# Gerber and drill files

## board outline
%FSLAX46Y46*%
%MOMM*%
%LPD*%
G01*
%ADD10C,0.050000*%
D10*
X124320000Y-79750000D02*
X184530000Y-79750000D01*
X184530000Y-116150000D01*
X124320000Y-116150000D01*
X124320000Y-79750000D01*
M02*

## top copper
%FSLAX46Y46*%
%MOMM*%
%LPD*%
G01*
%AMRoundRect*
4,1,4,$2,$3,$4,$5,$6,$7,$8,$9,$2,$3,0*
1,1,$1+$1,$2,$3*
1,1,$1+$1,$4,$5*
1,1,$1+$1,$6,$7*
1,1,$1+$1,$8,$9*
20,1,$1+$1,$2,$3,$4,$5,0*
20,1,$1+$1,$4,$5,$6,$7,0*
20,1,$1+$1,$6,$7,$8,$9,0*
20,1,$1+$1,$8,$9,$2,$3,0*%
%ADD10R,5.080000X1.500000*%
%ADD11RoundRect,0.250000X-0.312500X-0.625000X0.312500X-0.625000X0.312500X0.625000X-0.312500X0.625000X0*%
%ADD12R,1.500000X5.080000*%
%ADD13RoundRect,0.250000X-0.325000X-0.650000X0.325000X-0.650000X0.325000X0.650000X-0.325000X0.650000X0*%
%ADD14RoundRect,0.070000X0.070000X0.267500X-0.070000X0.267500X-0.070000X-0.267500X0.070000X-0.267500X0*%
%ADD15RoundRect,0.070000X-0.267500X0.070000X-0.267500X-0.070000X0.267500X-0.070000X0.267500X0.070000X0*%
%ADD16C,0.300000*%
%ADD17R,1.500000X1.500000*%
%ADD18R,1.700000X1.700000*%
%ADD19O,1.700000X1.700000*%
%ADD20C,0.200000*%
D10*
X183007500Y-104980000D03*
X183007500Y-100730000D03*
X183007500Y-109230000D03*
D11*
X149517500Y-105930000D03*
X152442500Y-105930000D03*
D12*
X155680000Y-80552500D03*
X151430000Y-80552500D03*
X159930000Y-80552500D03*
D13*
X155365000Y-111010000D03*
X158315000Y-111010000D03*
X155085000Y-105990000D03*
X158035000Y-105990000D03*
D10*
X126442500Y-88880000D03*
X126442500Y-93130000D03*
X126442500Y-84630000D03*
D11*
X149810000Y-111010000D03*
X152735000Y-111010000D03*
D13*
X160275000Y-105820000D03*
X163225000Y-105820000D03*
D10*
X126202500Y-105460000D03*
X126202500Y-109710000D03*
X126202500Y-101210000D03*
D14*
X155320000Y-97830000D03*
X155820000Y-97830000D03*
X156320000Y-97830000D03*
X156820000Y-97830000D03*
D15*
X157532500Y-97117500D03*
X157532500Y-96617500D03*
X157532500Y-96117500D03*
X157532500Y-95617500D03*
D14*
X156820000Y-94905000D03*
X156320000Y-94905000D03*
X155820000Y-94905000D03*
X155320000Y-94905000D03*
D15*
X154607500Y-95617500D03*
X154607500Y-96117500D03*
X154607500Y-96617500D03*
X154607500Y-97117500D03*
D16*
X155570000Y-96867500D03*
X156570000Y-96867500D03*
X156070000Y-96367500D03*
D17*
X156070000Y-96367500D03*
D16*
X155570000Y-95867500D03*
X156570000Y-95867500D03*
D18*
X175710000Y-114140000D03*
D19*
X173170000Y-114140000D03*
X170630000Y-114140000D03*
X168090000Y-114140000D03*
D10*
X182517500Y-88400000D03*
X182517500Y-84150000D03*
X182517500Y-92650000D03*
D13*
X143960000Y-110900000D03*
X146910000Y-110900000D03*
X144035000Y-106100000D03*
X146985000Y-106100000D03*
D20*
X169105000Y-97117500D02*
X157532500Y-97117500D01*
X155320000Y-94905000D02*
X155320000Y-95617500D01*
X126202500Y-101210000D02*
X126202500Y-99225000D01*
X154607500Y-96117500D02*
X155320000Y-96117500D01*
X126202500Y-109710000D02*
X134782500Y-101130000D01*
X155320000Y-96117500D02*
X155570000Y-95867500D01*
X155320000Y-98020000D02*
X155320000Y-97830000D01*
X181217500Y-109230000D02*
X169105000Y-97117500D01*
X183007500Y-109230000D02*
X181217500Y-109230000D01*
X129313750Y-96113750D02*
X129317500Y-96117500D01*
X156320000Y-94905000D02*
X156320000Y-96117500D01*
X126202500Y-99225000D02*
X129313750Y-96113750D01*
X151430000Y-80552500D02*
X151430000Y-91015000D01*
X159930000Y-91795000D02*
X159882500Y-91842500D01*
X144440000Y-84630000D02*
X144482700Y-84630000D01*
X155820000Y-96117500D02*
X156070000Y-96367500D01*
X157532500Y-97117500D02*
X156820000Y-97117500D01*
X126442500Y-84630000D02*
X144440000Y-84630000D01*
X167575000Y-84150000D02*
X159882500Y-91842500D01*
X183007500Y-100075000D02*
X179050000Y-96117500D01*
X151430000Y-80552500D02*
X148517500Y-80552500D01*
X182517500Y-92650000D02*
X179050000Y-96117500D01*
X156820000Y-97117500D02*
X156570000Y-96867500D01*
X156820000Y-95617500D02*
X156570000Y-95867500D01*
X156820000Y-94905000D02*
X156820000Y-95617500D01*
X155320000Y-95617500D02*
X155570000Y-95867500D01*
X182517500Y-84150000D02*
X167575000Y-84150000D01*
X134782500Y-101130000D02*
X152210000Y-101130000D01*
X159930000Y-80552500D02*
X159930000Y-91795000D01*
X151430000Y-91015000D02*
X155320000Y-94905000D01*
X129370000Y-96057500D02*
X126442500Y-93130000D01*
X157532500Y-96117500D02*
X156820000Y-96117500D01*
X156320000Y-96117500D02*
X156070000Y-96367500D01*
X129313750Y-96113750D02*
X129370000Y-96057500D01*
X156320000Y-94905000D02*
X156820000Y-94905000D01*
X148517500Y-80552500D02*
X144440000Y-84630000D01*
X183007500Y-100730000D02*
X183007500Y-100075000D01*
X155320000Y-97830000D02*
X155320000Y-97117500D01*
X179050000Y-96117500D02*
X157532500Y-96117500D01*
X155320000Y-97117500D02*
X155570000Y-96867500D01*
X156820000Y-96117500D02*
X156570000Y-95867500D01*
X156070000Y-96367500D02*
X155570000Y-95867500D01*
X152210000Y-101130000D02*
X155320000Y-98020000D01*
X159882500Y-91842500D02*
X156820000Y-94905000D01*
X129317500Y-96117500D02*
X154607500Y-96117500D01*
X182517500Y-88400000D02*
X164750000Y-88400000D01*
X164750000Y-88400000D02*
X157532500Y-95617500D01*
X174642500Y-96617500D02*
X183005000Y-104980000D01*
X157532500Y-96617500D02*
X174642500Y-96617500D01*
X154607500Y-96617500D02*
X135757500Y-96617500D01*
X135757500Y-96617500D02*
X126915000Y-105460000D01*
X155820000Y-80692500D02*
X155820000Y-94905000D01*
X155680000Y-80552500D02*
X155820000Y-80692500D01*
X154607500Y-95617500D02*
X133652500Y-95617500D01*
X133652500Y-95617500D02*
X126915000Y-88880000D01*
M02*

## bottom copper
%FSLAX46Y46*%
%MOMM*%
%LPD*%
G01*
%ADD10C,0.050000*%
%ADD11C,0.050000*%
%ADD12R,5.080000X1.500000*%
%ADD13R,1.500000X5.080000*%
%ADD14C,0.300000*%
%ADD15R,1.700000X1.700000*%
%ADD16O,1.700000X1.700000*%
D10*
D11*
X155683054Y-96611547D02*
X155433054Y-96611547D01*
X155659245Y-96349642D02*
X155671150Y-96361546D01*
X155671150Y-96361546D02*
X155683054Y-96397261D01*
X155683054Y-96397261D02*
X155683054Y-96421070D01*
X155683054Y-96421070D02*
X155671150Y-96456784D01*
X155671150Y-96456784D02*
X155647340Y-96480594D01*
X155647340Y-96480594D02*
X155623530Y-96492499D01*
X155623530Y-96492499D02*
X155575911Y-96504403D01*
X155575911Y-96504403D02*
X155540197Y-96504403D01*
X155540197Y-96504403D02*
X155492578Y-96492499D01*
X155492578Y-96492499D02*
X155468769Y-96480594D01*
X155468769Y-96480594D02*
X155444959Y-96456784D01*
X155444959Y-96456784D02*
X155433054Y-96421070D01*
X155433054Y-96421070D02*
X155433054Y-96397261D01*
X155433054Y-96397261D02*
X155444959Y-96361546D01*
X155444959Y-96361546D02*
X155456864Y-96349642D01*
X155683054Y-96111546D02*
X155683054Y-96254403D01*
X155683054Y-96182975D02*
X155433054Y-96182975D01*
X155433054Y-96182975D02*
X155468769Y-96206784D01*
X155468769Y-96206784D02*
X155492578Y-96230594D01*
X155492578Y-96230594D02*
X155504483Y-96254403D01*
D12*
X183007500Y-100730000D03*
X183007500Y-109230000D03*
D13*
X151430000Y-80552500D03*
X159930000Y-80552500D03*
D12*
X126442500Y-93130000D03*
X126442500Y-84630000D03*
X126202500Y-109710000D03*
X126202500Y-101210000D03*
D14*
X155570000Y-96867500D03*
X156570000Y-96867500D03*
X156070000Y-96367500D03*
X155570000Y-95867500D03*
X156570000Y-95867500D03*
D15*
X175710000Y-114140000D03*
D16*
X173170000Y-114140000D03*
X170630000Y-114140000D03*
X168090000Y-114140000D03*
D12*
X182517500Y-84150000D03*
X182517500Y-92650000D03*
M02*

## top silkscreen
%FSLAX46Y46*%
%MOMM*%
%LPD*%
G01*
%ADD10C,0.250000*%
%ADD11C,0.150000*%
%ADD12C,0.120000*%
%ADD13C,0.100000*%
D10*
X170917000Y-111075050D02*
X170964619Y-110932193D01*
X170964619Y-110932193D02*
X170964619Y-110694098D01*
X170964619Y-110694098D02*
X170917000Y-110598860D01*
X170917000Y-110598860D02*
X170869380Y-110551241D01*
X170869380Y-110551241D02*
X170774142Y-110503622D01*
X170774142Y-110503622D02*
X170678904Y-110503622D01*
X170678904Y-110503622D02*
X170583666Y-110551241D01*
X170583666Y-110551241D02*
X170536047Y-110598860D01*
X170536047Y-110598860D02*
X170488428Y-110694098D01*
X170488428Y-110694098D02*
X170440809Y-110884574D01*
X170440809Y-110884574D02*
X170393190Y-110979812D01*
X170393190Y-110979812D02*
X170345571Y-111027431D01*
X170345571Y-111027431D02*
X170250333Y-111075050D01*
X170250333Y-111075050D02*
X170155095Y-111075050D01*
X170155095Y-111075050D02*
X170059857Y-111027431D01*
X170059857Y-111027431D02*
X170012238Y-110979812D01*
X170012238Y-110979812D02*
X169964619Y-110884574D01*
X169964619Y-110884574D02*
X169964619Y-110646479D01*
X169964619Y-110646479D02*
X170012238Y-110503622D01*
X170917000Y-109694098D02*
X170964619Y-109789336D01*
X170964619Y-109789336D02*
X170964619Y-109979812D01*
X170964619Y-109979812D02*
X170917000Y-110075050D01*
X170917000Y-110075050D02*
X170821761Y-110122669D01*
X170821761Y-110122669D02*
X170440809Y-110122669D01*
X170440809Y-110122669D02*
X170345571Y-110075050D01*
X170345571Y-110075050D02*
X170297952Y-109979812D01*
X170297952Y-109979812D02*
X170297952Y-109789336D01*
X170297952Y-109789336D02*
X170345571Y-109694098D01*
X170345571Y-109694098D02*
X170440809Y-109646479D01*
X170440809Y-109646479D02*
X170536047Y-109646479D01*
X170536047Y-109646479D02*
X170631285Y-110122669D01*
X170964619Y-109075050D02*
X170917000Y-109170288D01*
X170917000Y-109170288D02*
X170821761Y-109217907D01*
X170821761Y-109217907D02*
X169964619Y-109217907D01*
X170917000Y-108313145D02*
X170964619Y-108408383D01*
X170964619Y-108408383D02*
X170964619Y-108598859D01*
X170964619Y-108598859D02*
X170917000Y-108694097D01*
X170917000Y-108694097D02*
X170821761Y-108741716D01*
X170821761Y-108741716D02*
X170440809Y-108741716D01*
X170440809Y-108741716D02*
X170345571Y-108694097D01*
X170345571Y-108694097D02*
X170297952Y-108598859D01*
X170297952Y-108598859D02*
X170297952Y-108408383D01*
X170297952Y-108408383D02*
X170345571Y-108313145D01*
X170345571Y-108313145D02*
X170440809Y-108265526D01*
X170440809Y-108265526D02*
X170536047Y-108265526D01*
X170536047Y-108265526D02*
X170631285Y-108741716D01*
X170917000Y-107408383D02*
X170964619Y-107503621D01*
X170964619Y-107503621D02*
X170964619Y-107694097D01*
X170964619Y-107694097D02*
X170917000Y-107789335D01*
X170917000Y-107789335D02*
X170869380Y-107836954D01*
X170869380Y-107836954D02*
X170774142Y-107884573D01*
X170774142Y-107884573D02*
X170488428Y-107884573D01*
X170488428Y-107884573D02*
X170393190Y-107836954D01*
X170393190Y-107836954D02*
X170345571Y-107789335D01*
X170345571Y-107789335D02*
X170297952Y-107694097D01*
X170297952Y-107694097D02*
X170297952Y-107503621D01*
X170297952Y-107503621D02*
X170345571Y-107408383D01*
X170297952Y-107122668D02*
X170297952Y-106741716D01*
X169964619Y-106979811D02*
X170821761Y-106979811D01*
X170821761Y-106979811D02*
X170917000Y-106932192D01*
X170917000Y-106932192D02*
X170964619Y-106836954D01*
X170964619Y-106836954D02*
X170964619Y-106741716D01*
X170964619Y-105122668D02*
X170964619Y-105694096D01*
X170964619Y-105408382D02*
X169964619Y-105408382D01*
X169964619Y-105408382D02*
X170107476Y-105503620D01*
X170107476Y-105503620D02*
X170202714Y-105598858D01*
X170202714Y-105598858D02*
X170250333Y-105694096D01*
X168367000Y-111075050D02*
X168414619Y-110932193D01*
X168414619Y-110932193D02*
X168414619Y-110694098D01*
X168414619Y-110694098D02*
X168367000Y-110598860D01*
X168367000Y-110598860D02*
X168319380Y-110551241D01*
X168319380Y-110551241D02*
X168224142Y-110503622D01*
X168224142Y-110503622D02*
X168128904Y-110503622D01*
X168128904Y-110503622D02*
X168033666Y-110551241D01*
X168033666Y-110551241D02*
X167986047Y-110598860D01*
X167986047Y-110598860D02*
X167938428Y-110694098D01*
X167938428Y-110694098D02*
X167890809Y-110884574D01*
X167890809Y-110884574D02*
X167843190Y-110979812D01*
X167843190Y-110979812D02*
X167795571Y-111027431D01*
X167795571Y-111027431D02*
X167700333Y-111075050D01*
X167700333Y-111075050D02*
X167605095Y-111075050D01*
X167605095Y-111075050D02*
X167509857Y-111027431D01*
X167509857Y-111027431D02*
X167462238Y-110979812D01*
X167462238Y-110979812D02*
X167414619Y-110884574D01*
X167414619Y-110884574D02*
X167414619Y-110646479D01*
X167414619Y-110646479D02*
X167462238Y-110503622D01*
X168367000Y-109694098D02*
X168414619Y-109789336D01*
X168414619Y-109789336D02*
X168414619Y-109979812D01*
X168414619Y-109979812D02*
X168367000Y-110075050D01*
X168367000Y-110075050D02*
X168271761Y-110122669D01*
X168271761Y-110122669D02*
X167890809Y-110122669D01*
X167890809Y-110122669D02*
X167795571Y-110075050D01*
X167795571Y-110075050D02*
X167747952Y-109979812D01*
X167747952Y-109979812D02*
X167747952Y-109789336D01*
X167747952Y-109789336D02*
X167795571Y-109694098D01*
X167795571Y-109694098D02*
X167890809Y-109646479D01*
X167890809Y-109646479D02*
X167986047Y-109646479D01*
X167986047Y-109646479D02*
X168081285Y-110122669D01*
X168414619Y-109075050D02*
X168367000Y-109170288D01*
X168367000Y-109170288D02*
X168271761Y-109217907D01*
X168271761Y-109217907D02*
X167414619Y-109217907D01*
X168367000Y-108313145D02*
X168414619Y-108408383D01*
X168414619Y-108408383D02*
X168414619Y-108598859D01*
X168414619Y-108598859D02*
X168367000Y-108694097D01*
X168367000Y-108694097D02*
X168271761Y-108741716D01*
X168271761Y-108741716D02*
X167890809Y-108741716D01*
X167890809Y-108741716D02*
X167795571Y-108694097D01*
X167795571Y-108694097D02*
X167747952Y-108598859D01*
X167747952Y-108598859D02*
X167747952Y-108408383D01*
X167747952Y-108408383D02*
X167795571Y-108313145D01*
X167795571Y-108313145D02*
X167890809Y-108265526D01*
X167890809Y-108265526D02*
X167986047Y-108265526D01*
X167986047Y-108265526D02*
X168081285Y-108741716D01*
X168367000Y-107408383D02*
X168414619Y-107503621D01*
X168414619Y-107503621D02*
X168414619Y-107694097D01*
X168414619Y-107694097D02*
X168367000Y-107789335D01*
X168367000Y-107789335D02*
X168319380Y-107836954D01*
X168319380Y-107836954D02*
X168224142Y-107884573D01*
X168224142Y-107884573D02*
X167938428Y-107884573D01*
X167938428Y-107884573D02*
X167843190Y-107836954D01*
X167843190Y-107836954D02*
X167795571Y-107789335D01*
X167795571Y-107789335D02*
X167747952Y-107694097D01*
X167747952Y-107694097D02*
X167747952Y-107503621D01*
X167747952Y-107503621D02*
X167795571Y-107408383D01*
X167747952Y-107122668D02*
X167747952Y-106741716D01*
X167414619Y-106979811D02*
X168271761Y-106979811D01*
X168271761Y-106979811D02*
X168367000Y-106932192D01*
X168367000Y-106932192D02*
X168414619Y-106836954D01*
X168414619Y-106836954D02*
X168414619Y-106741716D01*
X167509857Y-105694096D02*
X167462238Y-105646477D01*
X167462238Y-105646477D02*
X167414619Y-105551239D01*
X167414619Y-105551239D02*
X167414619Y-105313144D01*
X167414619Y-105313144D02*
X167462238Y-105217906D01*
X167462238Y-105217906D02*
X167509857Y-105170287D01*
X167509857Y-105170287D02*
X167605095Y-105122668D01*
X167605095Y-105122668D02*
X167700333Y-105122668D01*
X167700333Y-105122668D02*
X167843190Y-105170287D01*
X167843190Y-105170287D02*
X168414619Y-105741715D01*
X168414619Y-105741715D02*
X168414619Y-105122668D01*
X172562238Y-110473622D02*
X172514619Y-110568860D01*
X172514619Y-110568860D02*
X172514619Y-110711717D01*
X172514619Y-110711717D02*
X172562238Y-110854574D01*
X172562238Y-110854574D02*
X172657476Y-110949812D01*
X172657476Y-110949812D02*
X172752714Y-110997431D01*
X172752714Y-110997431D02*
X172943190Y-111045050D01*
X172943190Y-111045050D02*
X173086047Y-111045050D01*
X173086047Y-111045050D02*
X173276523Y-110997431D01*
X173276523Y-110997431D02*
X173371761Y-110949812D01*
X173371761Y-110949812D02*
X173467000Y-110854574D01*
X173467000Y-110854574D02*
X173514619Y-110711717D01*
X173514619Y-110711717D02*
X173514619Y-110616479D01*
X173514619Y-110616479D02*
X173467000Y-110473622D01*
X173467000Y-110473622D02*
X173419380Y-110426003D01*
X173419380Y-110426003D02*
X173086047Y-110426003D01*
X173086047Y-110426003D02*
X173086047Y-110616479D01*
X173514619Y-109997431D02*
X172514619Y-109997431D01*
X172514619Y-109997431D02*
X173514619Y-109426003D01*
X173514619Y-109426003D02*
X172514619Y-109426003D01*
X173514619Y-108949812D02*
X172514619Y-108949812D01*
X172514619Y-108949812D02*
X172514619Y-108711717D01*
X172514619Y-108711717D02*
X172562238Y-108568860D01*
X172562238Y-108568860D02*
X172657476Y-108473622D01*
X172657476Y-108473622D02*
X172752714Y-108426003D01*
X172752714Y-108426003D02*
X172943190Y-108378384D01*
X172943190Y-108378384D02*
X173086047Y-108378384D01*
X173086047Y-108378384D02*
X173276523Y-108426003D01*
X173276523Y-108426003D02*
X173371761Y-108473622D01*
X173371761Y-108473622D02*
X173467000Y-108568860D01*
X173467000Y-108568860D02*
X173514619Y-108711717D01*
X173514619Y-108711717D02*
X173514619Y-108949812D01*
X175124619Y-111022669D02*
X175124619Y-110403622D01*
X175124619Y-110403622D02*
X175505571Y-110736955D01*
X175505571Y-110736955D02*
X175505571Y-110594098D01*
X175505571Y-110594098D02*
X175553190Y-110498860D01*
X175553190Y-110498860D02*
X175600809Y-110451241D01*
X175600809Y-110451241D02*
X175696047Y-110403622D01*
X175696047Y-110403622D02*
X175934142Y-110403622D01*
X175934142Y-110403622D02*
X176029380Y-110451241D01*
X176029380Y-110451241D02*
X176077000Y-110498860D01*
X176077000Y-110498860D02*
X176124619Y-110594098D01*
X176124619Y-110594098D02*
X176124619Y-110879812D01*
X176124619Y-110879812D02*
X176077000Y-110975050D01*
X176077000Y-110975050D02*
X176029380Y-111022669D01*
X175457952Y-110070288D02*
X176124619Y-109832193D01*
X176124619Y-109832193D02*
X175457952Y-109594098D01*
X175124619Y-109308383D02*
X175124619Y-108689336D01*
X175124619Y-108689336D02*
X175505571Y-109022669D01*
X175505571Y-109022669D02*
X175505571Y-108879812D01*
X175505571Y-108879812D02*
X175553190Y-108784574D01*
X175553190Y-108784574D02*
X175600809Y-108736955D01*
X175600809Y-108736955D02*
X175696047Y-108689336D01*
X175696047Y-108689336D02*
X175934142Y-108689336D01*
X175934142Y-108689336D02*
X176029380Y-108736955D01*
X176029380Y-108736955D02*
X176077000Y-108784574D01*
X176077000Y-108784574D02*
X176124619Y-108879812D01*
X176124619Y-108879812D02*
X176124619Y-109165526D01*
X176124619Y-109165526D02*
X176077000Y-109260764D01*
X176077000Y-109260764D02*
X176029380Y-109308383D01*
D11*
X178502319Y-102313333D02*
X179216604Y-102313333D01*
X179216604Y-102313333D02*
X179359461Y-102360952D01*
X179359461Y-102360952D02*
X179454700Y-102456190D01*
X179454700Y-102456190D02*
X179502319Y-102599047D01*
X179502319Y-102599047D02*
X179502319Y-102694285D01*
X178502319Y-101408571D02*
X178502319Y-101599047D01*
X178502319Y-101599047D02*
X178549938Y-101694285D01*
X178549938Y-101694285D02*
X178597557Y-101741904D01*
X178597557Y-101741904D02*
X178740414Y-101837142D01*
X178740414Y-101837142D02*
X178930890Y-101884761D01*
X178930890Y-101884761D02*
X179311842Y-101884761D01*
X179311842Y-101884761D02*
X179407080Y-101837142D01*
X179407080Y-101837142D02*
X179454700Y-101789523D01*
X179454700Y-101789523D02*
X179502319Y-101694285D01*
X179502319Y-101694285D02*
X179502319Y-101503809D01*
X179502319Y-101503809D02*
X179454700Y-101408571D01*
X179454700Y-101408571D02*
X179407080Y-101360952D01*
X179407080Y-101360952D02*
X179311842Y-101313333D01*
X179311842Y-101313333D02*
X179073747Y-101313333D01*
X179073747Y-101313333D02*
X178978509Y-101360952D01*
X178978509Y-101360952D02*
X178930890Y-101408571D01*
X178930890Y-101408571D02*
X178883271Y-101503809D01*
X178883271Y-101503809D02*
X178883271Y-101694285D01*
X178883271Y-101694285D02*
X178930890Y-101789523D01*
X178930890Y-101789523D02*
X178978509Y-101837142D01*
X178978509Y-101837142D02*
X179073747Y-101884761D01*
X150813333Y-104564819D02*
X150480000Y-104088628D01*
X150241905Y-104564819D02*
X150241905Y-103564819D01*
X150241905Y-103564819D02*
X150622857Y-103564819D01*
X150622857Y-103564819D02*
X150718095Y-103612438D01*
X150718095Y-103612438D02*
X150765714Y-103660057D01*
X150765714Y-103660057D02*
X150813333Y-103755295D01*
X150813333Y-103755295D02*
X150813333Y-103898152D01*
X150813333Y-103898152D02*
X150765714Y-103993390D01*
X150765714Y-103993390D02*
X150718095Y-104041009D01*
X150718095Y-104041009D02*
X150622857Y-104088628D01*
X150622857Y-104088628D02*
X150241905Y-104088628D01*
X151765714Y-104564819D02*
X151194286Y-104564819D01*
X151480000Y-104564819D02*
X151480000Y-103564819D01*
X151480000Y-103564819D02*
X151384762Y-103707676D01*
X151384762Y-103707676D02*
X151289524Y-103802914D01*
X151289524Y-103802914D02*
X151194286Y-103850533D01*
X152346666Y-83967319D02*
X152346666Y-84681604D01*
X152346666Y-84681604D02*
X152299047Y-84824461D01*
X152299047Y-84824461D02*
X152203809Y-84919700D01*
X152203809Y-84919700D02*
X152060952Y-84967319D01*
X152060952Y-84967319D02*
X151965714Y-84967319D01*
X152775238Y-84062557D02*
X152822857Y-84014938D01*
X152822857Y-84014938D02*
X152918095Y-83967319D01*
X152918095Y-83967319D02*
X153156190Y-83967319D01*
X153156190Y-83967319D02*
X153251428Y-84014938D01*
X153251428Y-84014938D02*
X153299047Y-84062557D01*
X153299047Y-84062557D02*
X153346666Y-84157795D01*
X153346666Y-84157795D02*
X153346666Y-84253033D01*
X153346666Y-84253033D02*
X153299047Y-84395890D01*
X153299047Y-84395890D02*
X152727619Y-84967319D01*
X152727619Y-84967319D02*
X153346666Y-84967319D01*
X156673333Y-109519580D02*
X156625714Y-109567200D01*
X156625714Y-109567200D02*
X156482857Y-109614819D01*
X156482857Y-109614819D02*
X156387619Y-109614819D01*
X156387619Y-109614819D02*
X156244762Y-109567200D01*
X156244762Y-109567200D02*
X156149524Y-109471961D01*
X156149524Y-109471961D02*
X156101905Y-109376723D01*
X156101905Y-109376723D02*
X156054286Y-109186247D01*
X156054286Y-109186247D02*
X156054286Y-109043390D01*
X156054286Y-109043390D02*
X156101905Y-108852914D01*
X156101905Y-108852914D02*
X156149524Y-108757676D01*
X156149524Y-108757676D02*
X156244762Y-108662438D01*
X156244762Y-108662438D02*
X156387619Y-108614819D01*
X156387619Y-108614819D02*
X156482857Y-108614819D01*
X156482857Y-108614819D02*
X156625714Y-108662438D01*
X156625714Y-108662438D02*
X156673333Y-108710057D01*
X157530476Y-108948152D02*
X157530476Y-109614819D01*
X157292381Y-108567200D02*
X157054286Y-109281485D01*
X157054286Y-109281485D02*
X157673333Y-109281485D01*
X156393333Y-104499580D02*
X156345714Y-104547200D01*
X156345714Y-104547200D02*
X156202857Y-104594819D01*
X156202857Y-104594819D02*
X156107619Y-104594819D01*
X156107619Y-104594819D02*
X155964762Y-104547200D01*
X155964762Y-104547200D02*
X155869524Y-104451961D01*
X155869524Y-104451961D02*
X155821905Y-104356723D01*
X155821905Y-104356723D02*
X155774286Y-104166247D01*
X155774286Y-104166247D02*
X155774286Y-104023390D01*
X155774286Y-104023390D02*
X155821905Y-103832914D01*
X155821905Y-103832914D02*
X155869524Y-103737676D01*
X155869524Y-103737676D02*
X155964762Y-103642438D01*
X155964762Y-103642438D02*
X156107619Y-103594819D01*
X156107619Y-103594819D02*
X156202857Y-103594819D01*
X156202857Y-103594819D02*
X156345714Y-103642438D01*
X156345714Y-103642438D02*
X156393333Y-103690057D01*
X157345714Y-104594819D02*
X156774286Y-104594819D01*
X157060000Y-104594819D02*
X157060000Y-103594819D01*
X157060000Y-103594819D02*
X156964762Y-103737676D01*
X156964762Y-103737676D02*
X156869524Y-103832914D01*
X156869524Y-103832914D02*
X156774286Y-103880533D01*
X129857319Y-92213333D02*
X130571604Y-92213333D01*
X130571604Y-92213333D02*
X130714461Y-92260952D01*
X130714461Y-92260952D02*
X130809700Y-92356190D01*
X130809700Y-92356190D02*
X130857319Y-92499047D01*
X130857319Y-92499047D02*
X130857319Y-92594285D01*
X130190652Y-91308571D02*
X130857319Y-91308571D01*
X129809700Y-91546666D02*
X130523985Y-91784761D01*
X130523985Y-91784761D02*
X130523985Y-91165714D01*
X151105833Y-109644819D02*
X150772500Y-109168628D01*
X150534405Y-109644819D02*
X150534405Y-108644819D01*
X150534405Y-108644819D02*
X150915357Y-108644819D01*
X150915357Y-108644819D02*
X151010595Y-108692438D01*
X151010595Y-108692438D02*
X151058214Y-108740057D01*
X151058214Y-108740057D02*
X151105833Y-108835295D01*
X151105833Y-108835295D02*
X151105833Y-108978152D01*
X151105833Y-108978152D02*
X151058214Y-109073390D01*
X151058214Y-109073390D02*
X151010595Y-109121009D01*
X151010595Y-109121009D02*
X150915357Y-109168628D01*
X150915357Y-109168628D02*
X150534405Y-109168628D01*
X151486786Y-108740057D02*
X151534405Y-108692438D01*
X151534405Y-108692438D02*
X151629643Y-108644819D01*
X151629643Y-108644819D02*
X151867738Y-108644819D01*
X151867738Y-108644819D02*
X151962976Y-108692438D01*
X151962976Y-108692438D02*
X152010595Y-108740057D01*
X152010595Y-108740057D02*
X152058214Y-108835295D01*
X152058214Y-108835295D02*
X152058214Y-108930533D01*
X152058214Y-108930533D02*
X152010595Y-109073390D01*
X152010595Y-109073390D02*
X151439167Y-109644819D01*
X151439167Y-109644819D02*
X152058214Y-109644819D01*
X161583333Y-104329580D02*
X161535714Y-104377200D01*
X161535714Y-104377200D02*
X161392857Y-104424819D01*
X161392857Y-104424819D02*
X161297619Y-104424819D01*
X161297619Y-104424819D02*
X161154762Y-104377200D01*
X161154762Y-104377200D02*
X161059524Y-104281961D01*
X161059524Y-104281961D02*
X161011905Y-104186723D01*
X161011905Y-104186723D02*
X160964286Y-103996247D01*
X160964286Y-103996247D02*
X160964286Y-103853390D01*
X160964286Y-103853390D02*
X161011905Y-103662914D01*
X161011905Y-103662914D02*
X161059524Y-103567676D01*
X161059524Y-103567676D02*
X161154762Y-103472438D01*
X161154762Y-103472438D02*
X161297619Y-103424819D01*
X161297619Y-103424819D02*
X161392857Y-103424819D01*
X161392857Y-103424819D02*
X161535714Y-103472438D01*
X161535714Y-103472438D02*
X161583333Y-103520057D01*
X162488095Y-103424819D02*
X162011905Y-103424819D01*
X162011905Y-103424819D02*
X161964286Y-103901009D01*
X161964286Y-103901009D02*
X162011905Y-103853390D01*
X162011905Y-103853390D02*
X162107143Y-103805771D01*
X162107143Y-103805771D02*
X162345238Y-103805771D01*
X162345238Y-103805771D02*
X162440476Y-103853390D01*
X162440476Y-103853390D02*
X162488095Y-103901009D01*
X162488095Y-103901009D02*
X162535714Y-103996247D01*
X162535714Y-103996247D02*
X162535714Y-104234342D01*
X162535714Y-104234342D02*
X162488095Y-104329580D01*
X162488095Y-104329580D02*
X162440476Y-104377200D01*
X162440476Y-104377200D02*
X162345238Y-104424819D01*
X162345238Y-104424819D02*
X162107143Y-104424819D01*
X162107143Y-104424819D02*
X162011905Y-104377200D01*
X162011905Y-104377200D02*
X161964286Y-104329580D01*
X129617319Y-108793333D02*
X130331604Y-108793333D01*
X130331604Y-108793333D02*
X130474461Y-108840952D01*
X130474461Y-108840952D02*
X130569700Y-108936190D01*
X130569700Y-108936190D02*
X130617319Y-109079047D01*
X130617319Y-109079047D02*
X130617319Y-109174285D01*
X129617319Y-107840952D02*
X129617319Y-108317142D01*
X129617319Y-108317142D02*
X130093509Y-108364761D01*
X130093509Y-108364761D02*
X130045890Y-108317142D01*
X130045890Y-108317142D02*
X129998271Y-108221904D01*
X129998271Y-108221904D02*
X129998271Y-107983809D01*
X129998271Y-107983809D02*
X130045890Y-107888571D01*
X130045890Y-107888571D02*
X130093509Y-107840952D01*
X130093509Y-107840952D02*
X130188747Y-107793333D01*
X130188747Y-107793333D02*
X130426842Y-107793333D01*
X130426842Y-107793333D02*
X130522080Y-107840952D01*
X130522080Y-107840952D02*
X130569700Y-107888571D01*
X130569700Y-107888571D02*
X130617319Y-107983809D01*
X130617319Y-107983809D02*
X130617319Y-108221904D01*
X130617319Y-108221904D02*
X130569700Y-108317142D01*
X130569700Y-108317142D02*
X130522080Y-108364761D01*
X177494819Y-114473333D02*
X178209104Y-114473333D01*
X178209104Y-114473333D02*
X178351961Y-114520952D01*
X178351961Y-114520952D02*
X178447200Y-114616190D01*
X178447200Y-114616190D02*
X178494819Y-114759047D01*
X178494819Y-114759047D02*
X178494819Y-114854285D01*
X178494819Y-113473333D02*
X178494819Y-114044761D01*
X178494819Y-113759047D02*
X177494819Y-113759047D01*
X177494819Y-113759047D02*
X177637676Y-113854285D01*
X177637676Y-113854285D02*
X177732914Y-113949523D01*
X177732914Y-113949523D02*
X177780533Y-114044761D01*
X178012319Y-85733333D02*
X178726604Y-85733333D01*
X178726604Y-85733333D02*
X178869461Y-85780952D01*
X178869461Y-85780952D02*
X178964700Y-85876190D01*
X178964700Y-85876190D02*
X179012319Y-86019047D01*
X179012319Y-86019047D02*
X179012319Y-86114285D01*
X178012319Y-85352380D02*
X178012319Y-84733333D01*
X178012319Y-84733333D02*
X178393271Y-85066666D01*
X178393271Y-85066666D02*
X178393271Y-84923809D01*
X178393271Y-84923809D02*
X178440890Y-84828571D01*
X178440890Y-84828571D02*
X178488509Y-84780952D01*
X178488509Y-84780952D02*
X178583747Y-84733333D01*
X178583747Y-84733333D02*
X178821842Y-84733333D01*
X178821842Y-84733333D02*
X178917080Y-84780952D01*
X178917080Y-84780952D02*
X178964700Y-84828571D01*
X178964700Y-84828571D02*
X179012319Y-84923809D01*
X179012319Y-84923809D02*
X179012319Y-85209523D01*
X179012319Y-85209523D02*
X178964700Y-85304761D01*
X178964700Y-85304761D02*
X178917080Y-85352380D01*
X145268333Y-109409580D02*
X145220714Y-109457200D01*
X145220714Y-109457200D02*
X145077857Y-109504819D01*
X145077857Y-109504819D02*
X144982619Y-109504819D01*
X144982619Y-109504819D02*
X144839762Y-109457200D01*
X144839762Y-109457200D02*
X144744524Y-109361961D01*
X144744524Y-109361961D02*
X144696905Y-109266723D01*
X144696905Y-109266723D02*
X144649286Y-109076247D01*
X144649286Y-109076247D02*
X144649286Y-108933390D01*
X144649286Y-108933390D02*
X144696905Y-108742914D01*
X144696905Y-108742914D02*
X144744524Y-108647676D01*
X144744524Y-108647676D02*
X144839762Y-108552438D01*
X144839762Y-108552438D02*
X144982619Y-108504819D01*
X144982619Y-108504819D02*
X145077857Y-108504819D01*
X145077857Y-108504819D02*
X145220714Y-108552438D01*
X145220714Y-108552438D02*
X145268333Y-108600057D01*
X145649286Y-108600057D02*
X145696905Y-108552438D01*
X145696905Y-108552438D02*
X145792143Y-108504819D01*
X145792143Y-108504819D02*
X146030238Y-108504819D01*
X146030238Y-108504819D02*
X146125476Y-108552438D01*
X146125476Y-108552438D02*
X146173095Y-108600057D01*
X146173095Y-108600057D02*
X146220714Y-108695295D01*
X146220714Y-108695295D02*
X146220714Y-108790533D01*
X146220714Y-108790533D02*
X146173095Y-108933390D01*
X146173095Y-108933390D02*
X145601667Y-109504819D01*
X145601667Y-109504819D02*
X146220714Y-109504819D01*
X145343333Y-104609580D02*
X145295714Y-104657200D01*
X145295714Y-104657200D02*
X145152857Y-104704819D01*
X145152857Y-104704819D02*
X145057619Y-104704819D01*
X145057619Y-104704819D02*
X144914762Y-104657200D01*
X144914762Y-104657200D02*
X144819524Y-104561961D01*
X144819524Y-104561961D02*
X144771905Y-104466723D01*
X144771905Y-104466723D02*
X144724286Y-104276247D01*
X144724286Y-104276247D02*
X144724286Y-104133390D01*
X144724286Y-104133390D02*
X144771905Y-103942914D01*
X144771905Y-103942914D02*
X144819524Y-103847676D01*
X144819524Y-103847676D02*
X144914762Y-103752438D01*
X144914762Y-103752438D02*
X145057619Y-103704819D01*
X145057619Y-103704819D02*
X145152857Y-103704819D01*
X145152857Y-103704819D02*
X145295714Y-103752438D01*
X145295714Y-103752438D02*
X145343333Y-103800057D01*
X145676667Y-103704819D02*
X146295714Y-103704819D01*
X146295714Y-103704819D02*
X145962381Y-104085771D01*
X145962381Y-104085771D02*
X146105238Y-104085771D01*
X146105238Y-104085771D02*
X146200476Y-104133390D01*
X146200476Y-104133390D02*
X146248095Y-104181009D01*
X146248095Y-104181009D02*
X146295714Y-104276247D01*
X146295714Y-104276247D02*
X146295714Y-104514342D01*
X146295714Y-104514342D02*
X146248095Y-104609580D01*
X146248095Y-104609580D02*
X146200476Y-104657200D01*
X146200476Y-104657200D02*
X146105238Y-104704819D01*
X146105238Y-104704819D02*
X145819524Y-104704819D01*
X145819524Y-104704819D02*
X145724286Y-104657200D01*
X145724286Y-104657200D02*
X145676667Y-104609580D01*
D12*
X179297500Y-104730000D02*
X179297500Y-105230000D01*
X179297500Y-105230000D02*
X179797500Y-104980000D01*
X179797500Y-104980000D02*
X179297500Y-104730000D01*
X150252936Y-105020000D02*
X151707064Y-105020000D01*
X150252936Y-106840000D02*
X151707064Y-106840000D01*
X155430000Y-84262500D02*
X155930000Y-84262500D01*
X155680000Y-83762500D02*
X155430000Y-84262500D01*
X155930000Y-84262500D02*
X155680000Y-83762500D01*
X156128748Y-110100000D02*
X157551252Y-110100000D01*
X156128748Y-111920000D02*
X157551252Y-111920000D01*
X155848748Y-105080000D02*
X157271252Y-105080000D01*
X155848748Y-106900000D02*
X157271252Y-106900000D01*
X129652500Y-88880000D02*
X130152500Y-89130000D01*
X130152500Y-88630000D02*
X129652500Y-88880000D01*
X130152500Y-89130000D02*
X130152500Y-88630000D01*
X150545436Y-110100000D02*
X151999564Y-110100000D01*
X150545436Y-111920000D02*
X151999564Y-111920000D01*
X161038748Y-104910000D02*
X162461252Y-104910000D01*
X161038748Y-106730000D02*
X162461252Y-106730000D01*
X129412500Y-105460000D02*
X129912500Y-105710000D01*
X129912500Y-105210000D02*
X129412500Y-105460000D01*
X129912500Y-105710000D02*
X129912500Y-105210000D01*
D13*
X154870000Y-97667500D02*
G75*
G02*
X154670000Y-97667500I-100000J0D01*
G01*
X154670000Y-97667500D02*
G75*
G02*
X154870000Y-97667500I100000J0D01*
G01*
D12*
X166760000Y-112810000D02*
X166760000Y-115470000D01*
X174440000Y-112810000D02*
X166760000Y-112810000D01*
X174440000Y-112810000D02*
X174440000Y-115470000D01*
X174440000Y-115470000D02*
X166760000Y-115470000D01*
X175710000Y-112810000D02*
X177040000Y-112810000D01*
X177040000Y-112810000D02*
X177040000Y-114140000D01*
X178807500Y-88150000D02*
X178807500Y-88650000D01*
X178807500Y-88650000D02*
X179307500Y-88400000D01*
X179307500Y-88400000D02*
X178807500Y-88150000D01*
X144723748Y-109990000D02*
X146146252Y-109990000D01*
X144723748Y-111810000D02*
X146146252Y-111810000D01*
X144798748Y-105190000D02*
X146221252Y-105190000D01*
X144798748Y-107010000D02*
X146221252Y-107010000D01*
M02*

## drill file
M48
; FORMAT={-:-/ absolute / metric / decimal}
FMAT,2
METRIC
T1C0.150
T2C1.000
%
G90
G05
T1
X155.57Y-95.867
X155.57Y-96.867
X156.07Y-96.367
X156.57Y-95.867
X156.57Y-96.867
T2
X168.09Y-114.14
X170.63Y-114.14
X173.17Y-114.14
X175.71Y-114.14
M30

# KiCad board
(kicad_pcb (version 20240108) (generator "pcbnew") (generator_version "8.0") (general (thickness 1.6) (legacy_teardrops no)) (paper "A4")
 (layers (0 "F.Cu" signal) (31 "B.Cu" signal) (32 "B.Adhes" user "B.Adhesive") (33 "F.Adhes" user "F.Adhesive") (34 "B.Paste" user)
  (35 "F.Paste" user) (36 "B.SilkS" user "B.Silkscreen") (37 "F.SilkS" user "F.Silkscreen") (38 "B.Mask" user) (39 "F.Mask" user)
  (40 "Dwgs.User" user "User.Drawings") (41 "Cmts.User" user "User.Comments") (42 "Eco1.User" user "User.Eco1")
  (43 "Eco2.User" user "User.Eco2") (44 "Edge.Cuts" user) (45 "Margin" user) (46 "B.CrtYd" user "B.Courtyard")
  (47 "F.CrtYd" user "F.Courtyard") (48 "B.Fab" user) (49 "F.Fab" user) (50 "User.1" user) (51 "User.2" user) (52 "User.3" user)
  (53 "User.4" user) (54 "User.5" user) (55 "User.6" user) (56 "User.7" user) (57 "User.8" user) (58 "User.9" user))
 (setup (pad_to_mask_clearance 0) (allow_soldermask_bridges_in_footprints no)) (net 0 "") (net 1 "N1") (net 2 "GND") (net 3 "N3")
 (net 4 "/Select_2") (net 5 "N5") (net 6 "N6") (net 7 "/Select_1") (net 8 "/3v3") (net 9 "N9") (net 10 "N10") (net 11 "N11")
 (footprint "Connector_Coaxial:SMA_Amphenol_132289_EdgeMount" (layer "F.Cu") (at 183.0075 104.98)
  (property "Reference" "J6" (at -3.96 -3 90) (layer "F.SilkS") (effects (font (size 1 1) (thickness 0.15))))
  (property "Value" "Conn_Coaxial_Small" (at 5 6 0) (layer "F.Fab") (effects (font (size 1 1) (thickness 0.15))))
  (fp_line (start -3.71 -0.25) (end -3.71 0.25) (stroke (width 0.12) (type solid)) (layer "F.SilkS"))
  (fp_line (start -3.71 0.25) (end -3.21 0) (stroke (width 0.12) (type solid)) (layer "F.SilkS"))
  (fp_line (start -3.21 0) (end -3.71 -0.25) (stroke (width 0.12) (type solid)) (layer "F.SilkS"))
  (pad "1" smd rect (at 0 0 90) (size 1.5 5.08) (layers "F.Cu" "F.Paste" "F.Mask") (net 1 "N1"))
  (pad "2" smd rect (at 0 -4.25 90) (size 1.5 5.08) (layers "F.Cu" "F.Paste" "F.Mask") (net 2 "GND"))
  (pad "2" smd rect (at 0 -4.25 90) (size 1.5 5.08) (layers "B.Cu" "B.Paste" "B.Mask") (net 2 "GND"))
  (pad "2" smd rect (at 0 4.25 90) (size 1.5 5.08) (layers "F.Cu" "F.Paste" "F.Mask") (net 2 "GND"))
  (pad "2" smd rect (at 0 4.25 90) (size 1.5 5.08) (layers "B.Cu" "B.Paste" "B.Mask") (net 2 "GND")))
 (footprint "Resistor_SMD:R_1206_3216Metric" (layer "F.Cu") (at 150.98 105.93)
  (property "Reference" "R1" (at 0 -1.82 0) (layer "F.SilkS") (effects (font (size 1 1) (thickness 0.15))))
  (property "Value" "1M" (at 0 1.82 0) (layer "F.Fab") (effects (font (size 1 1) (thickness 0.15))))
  (fp_line (start -0.727064 -0.91) (end 0.727064 -0.91) (stroke (width 0.12) (type solid)) (layer "F.SilkS"))
  (fp_line (start -0.727064 0.91) (end 0.727064 0.91) (stroke (width 0.12) (type solid)) (layer "F.SilkS"))
  (pad "1" smd roundrect (at -1.4625 0) (size 1.125 1.75) (layers "F.Cu" "F.Paste" "F.Mask") (roundrect_rratio 0.222222) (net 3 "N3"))
  (pad "2" smd roundrect (at 1.4625 0) (size 1.125 1.75) (layers "F.Cu" "F.Paste" "F.Mask") (roundrect_rratio 0.222222) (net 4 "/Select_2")))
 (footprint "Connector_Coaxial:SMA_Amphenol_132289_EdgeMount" (layer "F.Cu") (at 155.68 80.5525 90)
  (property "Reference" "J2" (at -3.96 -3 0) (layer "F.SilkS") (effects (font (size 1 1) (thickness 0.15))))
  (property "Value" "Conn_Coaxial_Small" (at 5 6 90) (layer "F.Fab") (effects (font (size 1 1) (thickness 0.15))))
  (fp_line (start -3.71 -0.25) (end -3.71 0.25) (stroke (width 0.12) (type solid)) (layer "F.SilkS"))
  (fp_line (start -3.21 0) (end -3.71 -0.25) (stroke (width 0.12) (type solid)) (layer "F.SilkS"))
  (fp_line (start -3.71 0.25) (end -3.21 0) (stroke (width 0.12) (type solid)) (layer "F.SilkS"))
  (pad "1" smd rect (at 0 0 180) (size 1.5 5.08) (layers "F.Cu" "F.Paste" "F.Mask") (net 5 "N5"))
  (pad "2" smd rect (at 0 -4.25 180) (size 1.5 5.08) (layers "F.Cu" "F.Paste" "F.Mask") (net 2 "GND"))
  (pad "2" smd rect (at 0 -4.25 180) (size 1.5 5.08) (layers "B.Cu" "B.Paste" "B.Mask") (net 2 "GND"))
  (pad "2" smd rect (at 0 4.25 180) (size 1.5 5.08) (layers "F.Cu" "F.Paste" "F.Mask") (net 2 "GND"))
  (pad "2" smd rect (at 0 4.25 180) (size 1.5 5.08) (layers "B.Cu" "B.Paste" "B.Mask") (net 2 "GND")))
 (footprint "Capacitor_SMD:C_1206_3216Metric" (layer "F.Cu") (at 156.84 111.01)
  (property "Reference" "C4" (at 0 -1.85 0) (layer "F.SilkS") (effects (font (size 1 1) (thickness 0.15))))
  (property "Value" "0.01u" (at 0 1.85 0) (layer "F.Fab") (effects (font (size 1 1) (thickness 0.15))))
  (fp_line (start -0.711252 -0.91) (end 0.711252 -0.91) (stroke (width 0.12) (type solid)) (layer "F.SilkS"))
  (fp_line (start -0.711252 0.91) (end 0.711252 0.91) (stroke (width 0.12) (type solid)) (layer "F.SilkS"))
  (pad "1" smd roundrect (at -1.475 0) (size 1.15 1.8) (layers "F.Cu" "F.Paste" "F.Mask") (roundrect_rratio 0.217391) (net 2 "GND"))
  (pad "2" smd roundrect (at 1.475 0) (size 1.15 1.8) (layers "F.Cu" "F.Paste" "F.Mask") (roundrect_rratio 0.217391) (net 2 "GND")))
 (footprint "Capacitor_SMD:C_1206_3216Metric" (layer "F.Cu") (at 156.56 105.99)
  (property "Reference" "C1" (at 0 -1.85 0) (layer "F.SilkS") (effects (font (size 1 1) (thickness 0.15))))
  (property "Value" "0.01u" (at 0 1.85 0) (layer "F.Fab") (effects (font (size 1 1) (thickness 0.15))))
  (fp_line (start -0.711252 -0.91) (end 0.711252 -0.91) (stroke (width 0.12) (type solid)) (layer "F.SilkS"))
  (fp_line (start -0.711252 0.91) (end 0.711252 0.91) (stroke (width 0.12) (type solid)) (layer "F.SilkS"))
  (pad "1" smd roundrect (at -1.475 0) (size 1.15 1.8) (layers "F.Cu" "F.Paste" "F.Mask") (roundrect_rratio 0.217391) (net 4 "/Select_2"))
  (pad "2" smd roundrect (at 1.475 0) (size 1.15 1.8) (layers "F.Cu" "F.Paste" "F.Mask") (roundrect_rratio 0.217391) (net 2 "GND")))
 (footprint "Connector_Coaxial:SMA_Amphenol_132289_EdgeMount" (layer "F.Cu") (at 126.4425 88.88 180)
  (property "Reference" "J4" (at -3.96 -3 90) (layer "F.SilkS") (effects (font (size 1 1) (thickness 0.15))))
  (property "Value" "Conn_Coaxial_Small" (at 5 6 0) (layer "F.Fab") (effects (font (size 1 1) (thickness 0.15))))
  (fp_line (start -3.21 0) (end -3.71 -0.25) (stroke (width 0.12) (type solid)) (layer "F.SilkS"))
  (fp_line (start -3.71 0.25) (end -3.21 0) (stroke (width 0.12) (type solid)) (layer "F.SilkS"))
  (fp_line (start -3.71 -0.25) (end -3.71 0.25) (stroke (width 0.12) (type solid)) (layer "F.SilkS"))
  (pad "1" smd rect (at 0 0 270) (size 1.5 5.08) (layers "F.Cu" "F.Paste" "F.Mask") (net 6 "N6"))
  (pad "2" smd rect (at 0 -4.25 270) (size 1.5 5.08) (layers "F.Cu" "F.Paste" "F.Mask") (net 2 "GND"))
  (pad "2" smd rect (at 0 -4.25 270) (size 1.5 5.08) (layers "B.Cu" "B.Paste" "B.Mask") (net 2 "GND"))
  (pad "2" smd rect (at 0 4.25 270) (size 1.5 5.08) (layers "F.Cu" "F.Paste" "F.Mask") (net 2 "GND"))
  (pad "2" smd rect (at 0 4.25 270) (size 1.5 5.08) (layers "B.Cu" "B.Paste" "B.Mask") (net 2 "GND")))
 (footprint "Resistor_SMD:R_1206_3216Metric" (layer "F.Cu") (at 151.2725 111.01)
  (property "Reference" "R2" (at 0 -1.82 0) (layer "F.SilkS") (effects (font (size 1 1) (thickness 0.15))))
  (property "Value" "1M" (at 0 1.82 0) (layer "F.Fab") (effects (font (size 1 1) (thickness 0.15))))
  (fp_line (start -0.727064 -0.91) (end 0.727064 -0.91) (stroke (width 0.12) (type solid)) (layer "F.SilkS"))
  (fp_line (start -0.727064 0.91) (end 0.727064 0.91) (stroke (width 0.12) (type solid)) (layer "F.SilkS"))
  (pad "1" smd roundrect (at -1.4625 0) (size 1.125 1.75) (layers "F.Cu" "F.Paste" "F.Mask") (roundrect_rratio 0.222222) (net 3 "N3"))
  (pad "2" smd roundrect (at 1.4625 0) (size 1.125 1.75) (layers "F.Cu" "F.Paste" "F.Mask") (roundrect_rratio 0.222222) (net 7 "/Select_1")))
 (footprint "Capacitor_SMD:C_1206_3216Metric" (layer "F.Cu") (at 161.75 105.82)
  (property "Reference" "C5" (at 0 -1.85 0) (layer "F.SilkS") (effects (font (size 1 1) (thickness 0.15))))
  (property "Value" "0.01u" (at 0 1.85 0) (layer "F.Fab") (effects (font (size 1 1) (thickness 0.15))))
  (fp_line (start -0.711252 -0.91) (end 0.711252 -0.91) (stroke (width 0.12) (type solid)) (layer "F.SilkS"))
  (fp_line (start -0.711252 0.91) (end 0.711252 0.91) (stroke (width 0.12) (type solid)) (layer "F.SilkS"))
  (pad "1" smd roundrect (at -1.475 0) (size 1.15 1.8) (layers "F.Cu" "F.Paste" "F.Mask") (roundrect_rratio 0.217391) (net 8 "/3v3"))
  (pad "2" smd roundrect (at 1.475 0) (size 1.15 1.8) (layers "F.Cu" "F.Paste" "F.Mask") (roundrect_rratio 0.217391) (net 3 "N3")))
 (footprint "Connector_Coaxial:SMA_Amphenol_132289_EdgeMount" (layer "F.Cu") (at 126.2025 105.46 180)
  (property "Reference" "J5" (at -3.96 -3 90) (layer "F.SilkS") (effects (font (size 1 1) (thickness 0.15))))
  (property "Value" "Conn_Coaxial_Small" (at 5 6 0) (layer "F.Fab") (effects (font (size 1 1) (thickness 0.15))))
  (fp_line (start -3.21 0) (end -3.71 -0.25) (stroke (width 0.12) (type solid)) (layer "F.SilkS"))
  (fp_line (start -3.71 0.25) (end -3.21 0) (stroke (width 0.12) (type solid)) (layer "F.SilkS"))
  (fp_line (start -3.71 -0.25) (end -3.71 0.25) (stroke (width 0.12) (type solid)) (layer "F.SilkS"))
  (pad "1" smd rect (at 0 0 270) (size 1.5 5.08) (layers "F.Cu" "F.Paste" "F.Mask") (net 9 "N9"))
  (pad "2" smd rect (at 0 -4.25 270) (size 1.5 5.08) (layers "F.Cu" "F.Paste" "F.Mask") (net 2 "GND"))
  (pad "2" smd rect (at 0 -4.25 270) (size 1.5 5.08) (layers "B.Cu" "B.Paste" "B.Mask") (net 2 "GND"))
  (pad "2" smd rect (at 0 4.25 270) (size 1.5 5.08) (layers "F.Cu" "F.Paste" "F.Mask") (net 2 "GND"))
  (pad "2" smd rect (at 0 4.25 270) (size 1.5 5.08) (layers "B.Cu" "B.Paste" "B.Mask") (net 2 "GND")))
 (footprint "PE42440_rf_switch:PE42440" (layer "F.Cu") (at 156.07 96.3675 90)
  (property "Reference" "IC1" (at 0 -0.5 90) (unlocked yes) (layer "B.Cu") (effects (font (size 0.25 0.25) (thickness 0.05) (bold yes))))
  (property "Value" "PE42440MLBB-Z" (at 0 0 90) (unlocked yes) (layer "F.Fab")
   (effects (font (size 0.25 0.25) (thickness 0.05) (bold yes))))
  (fp_circle (center -1.3 -1.3) (end -1.2 -1.3) (stroke (width 0.1) (type default)) (fill none) (layer "F.SilkS"))
  (pad "1" smd roundrect (at -1.4625 -0.75 180) (size 0.28 0.675) (layers "F.Cu" "F.Paste" "F.Mask") (roundrect_rratio 0.25) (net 2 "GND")
   (thermal_bridge_angle 45))
  (pad "2" smd roundrect (at -1.4625 -0.25 180) (size 0.28 0.675) (layers "F.Cu" "F.Paste" "F.Mask") (roundrect_rratio 0.25) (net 8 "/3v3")
   (thermal_bridge_angle 45))
  (pad "3" smd roundrect (at -1.4625 0.25 180) (size 0.28 0.675) (layers "F.Cu" "F.Paste" "F.Mask") (roundrect_rratio 0.25)
   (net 4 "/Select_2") (thermal_bridge_angle 45))
  (pad "4" smd roundrect (at -1.4625 0.75 180) (size 0.28 0.675) (layers "F.Cu" "F.Paste" "F.Mask") (roundrect_rratio 0.25)
   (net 7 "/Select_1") (thermal_bridge_angle 45))
  (pad "5" smd roundrect (at -0.75 1.4625 270) (size 0.28 0.675) (layers "F.Cu" "F.Paste" "F.Mask") (roundrect_rratio 0.25) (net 2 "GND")
   (thermal_bridge_angle 45))
  (pad "6" smd roundrect (at -0.25 1.4625 270) (size 0.28 0.675) (layers "F.Cu" "F.Paste" "F.Mask") (roundrect_rratio 0.25) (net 1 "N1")
   (thermal_bridge_angle 45))
  (pad "7" smd roundrect (at 0.25 1.4625 270) (size 0.28 0.675) (layers "F.Cu" "F.Paste" "F.Mask") (roundrect_rratio 0.25) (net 2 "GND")
   (thermal_bridge_angle 45))
  (pad "8" smd roundrect (at 0.75 1.4625 270) (size 0.28 0.675) (layers "F.Cu" "F.Paste" "F.Mask") (roundrect_rratio 0.25) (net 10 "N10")
   (thermal_bridge_angle 45))
  (pad "9" smd roundrect (at 1.4625 0.75 180) (size 0.28 0.675) (layers "F.Cu" "F.Paste" "F.Mask") (roundrect_rratio 0.25) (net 2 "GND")
   (thermal_bridge_angle 45))
  (pad "10" smd roundrect (at 1.4625 0.25 180) (size 0.28 0.675) (layers "F.Cu" "F.Paste" "F.Mask") (roundrect_rratio 0.25) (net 2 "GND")
   (thermal_bridge_angle 45))
  (pad "11" smd roundrect (at 1.4625 -0.25 180) (size 0.28 0.675) (layers "F.Cu" "F.Paste" "F.Mask") (roundrect_rratio 0.25) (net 5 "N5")
   (thermal_bridge_angle 45))
  (pad "12" smd roundrect (at 1.4625 -0.75 180) (size 0.28 0.675) (layers "F.Cu" "F.Paste" "F.Mask") (roundrect_rratio 0.25) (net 2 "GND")
   (thermal_bridge_angle 45))
  (pad "13" smd roundrect (at 0.75 -1.4625 270) (size 0.28 0.675) (layers "F.Cu" "F.Paste" "F.Mask") (roundrect_rratio 0.25) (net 6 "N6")
   (thermal_bridge_angle 45))
  (pad "14" smd roundrect (at 0.25 -1.4625 270) (size 0.28 0.675) (layers "F.Cu" "F.Paste" "F.Mask") (roundrect_rratio 0.25) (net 2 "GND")
   (thermal_bridge_angle 45))
  (pad "15" smd roundrect (at -0.25 -1.4625 270) (size 0.28 0.675) (layers "F.Cu" "F.Paste" "F.Mask") (roundrect_rratio 0.25) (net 9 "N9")
   (thermal_bridge_angle 45))
  (pad "16" smd roundrect (at -0.75 -1.4625 270) (size 0.28 0.675) (layers "F.Cu" "F.Paste" "F.Mask") (roundrect_rratio 0.25) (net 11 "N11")
   (thermal_bridge_angle 45))
  (pad "17" thru_hole circle (at -0.5 -0.5 90) (size 0.3 0.3) (drill 0.15) (layers "*.Cu" "*.Mask") (remove_unused_layers no) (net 2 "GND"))
  (pad "17" thru_hole circle (at -0.5 0.5 90) (size 0.3 0.3) (drill 0.15) (layers "*.Cu" "*.Mask") (remove_unused_layers no) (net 2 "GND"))
  (pad "17" thru_hole circle (at 0 0 90) (size 0.3 0.3) (drill 0.15) (layers "*.Cu" "*.Mask") (remove_unused_layers no) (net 2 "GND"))
  (pad "17" smd rect (at 0 0 90) (size 1.5 1.5) (layers "F.Cu" "F.Paste" "F.Mask") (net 2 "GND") (thermal_bridge_angle 45))
  (pad "17" thru_hole circle (at 0.5 -0.5 90) (size 0.3 0.3) (drill 0.15) (layers "*.Cu" "*.Mask") (remove_unused_layers no) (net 2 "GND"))
  (pad "17" thru_hole circle (at 0.5 0.5 90) (size 0.3 0.3) (drill 0.15) (layers "*.Cu" "*.Mask") (remove_unused_layers no) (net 2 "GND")))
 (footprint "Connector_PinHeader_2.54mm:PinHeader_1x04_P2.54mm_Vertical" (layer "F.Cu") (at 175.71 114.14 -90)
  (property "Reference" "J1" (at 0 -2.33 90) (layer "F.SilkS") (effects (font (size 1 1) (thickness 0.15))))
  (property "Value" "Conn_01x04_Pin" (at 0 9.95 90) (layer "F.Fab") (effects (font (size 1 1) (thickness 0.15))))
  (fp_line (start -1.33 8.95) (end 1.33 8.95) (stroke (width 0.12) (type solid)) (layer "F.SilkS"))
  (fp_line (start -1.33 1.27) (end -1.33 8.95) (stroke (width 0.12) (type solid)) (layer "F.SilkS"))
  (fp_line (start -1.33 1.27) (end 1.33 1.27) (stroke (width 0.12) (type solid)) (layer "F.SilkS"))
  (fp_line (start 1.33 1.27) (end 1.33 8.95) (stroke (width 0.12) (type solid)) (layer "F.SilkS"))
  (fp_line (start -1.33 0) (end -1.33 -1.33) (stroke (width 0.12) (type solid)) (layer "F.SilkS"))
  (fp_line (start -1.33 -1.33) (end 0 -1.33) (stroke (width 0.12) (type solid)) (layer "F.SilkS"))
  (pad "1" thru_hole rect (at 0 0 270) (size 1.7 1.7) (drill 1) (layers "*.Cu" "*.Mask") (remove_unused_layers no) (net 8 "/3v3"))
  (pad "2" thru_hole oval (at 0 2.54 270) (size 1.7 1.7) (drill 1) (layers "*.Cu" "*.Mask") (remove_unused_layers no) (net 2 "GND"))
  (pad "3" thru_hole oval (at 0 5.08 270) (size 1.7 1.7) (drill 1) (layers "*.Cu" "*.Mask") (remove_unused_layers no) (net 7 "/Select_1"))
  (pad "4" thru_hole oval (at 0 7.62 270) (size 1.7 1.7) (drill 1) (layers "*.Cu" "*.Mask") (remove_unused_layers no) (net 4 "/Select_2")))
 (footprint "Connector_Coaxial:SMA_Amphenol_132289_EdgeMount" (layer "F.Cu") (at 182.5175 88.4)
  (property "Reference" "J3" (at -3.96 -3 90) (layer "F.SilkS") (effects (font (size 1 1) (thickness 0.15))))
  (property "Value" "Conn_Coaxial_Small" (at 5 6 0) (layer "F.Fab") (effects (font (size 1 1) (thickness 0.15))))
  (fp_line (start -3.71 -0.25) (end -3.71 0.25) (stroke (width 0.12) (type solid)) (layer "F.SilkS"))
  (fp_line (start -3.71 0.25) (end -3.21 0) (stroke (width 0.12) (type solid)) (layer "F.SilkS"))
  (fp_line (start -3.21 0) (end -3.71 -0.25) (stroke (width 0.12) (type solid)) (layer "F.SilkS"))
  (pad "1" smd rect (at 0 0 90) (size 1.5 5.08) (layers "F.Cu" "F.Paste" "F.Mask") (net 10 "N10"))
  (pad "2" smd rect (at 0 -4.25 90) (size 1.5 5.08) (layers "F.Cu" "F.Paste" "F.Mask") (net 2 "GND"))
  (pad "2" smd rect (at 0 -4.25 90) (size 1.5 5.08) (layers "B.Cu" "B.Paste" "B.Mask") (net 2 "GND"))
  (pad "2" smd rect (at 0 4.25 90) (size 1.5 5.08) (layers "F.Cu" "F.Paste" "F.Mask") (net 2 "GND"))
  (pad "2" smd rect (at 0 4.25 90) (size 1.5 5.08) (layers "B.Cu" "B.Paste" "B.Mask") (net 2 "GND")))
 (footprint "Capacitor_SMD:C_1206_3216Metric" (layer "F.Cu") (at 145.435 110.9)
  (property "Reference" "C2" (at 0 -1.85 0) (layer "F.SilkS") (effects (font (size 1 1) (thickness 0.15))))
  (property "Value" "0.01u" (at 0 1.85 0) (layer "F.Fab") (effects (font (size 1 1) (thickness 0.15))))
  (fp_line (start -0.711252 -0.91) (end 0.711252 -0.91) (stroke (width 0.12) (type solid)) (layer "F.SilkS"))
  (fp_line (start -0.711252 0.91) (end 0.711252 0.91) (stroke (width 0.12) (type solid)) (layer "F.SilkS"))
  (pad "1" smd roundrect (at -1.475 0) (size 1.15 1.8) (layers "F.Cu" "F.Paste" "F.Mask") (roundrect_rratio 0.217391) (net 7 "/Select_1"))
  (pad "2" smd roundrect (at 1.475 0) (size 1.15 1.8) (layers "F.Cu" "F.Paste" "F.Mask") (roundrect_rratio 0.217391) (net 2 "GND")))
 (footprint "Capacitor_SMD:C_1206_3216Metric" (layer "F.Cu") (at 145.51 106.1)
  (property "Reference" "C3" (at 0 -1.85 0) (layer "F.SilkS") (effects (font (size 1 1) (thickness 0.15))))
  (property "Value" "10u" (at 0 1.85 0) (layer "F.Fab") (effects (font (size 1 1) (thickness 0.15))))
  (fp_line (start -0.711252 -0.91) (end 0.711252 -0.91) (stroke (width 0.12) (type solid)) (layer "F.SilkS"))
  (fp_line (start -0.711252 0.91) (end 0.711252 0.91) (stroke (width 0.12) (type solid)) (layer "F.SilkS"))
  (pad "1" smd roundrect (at -1.475 0) (size 1.15 1.8) (layers "F.Cu" "F.Paste" "F.Mask") (roundrect_rratio 0.217391) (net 3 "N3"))
  (pad "2" smd roundrect (at 1.475 0) (size 1.15 1.8) (layers "F.Cu" "F.Paste" "F.Mask") (roundrect_rratio 0.217391) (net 2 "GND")))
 (gr_rect (start 124.32 79.75) (end 184.53 116.15) (stroke (width 0.05) (type default)) (fill none) (layer "Edge.Cuts"))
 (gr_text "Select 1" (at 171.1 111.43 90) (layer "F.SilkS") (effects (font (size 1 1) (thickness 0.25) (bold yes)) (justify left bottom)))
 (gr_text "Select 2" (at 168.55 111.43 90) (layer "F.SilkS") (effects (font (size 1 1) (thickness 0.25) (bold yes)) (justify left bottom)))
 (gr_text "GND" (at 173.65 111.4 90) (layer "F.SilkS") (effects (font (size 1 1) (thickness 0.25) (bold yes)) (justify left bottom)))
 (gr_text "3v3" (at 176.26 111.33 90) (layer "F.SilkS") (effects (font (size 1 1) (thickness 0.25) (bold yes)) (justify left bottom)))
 (segment (start 169.105 97.1175) (end 157.5325 97.1175) (width 0.2) (layer "F.Cu") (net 2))
 (segment (start 155.32 94.905) (end 155.32 95.6175) (width 0.2) (layer "F.Cu") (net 2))
 (segment (start 126.2025 101.21) (end 126.2025 99.225) (width 0.2) (layer "F.Cu") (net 2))
 (segment (start 154.6075 96.1175) (end 155.32 96.1175) (width 0.2) (layer "F.Cu") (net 2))
 (segment (start 126.2025 109.71) (end 134.7825 101.13) (width 0.2) (layer "F.Cu") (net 2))
 (segment (start 155.32 96.1175) (end 155.57 95.8675) (width 0.2) (layer "F.Cu") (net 2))
 (segment (start 155.32 98.02) (end 155.32 97.83) (width 0.2) (layer "F.Cu") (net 2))
 (segment (start 181.2175 109.23) (end 169.105 97.1175) (width 0.2) (layer "F.Cu") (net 2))
 (segment (start 183.0075 109.23) (end 181.2175 109.23) (width 0.2) (layer "F.Cu") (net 2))
 (segment (start 129.31375 96.11375) (end 129.3175 96.1175) (width 0.2) (layer "F.Cu") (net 2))
 (segment (start 156.32 94.905) (end 156.32 96.1175) (width 0.2) (layer "F.Cu") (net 2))
 (segment (start 126.2025 99.225) (end 129.31375 96.11375) (width 0.2) (layer "F.Cu") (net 2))
 (segment (start 151.43 80.5525) (end 151.43 91.015) (width 0.2) (layer "F.Cu") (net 2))
 (segment (start 159.93 91.795) (end 159.8825 91.8425) (width 0.2) (layer "F.Cu") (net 2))
 (segment (start 144.44 84.63) (end 144.4827 84.63) (width 0.2) (layer "F.Cu") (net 2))
 (segment (start 155.82 96.1175) (end 156.07 96.3675) (width 0.2) (layer "F.Cu") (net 2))
 (segment (start 157.5325 97.1175) (end 156.82 97.1175) (width 0.2) (layer "F.Cu") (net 2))
 (segment (start 126.4425 84.63) (end 144.44 84.63) (width 0.2) (layer "F.Cu") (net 2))
 (segment (start 167.575 84.15) (end 159.8825 91.8425) (width 0.2) (layer "F.Cu") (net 2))
 (segment (start 183.0075 100.075) (end 179.05 96.1175) (width 0.2) (layer "F.Cu") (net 2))
 (segment (start 151.43 80.5525) (end 148.5175 80.5525) (width 0.2) (layer "F.Cu") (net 2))
 (segment (start 182.5175 92.65) (end 179.05 96.1175) (width 0.2) (layer "F.Cu") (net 2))
 (segment (start 156.82 97.1175) (end 156.57 96.8675) (width 0.2) (layer "F.Cu") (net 2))
 (segment (start 156.82 95.6175) (end 156.57 95.8675) (width 0.2) (layer "F.Cu") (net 2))
 (segment (start 156.82 94.905) (end 156.82 95.6175) (width 0.2) (layer "F.Cu") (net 2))
 (segment (start 155.32 95.6175) (end 155.57 95.8675) (width 0.2) (layer "F.Cu") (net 2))
 (segment (start 182.5175 84.15) (end 167.575 84.15) (width 0.2) (layer "F.Cu") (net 2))
 (segment (start 134.7825 101.13) (end 152.21 101.13) (width 0.2) (layer "F.Cu") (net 2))
 (segment (start 159.93 80.5525) (end 159.93 91.795) (width 0.2) (layer "F.Cu") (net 2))
 (segment (start 151.43 91.015) (end 155.32 94.905) (width 0.2) (layer "F.Cu") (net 2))
 (segment (start 129.37 96.0575) (end 126.4425 93.13) (width 0.2) (layer "F.Cu") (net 2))
 (segment (start 157.5325 96.1175) (end 156.82 96.1175) (width 0.2) (layer "F.Cu") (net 2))
 (segment (start 156.32 96.1175) (end 156.07 96.3675) (width 0.2) (layer "F.Cu") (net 2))
 (segment (start 129.31375 96.11375) (end 129.37 96.0575) (width 0.2) (layer "F.Cu") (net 2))
 (segment (start 156.32 94.905) (end 156.82 94.905) (width 0.2) (layer "F.Cu") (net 2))
 (segment (start 148.5175 80.5525) (end 144.44 84.63) (width 0.2) (layer "F.Cu") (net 2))
 (segment (start 183.0075 100.73) (end 183.0075 100.075) (width 0.2) (layer "F.Cu") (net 2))
 (segment (start 155.32 97.83) (end 155.32 97.1175) (width 0.2) (layer "F.Cu") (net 2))
 (segment (start 179.05 96.1175) (end 157.5325 96.1175) (width 0.2) (layer "F.Cu") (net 2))
 (segment (start 155.32 97.1175) (end 155.57 96.8675) (width 0.2) (layer "F.Cu") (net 2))
 (segment (start 156.82 96.1175) (end 156.57 95.8675) (width 0.2) (layer "F.Cu") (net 2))
 (segment (start 156.07 96.3675) (end 155.57 95.8675) (width 0.2) (layer "F.Cu") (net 2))
 (segment (start 152.21 101.13) (end 155.32 98.02) (width 0.2) (layer "F.Cu") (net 2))
 (segment (start 159.8825 91.8425) (end 156.82 94.905) (width 0.2) (layer "F.Cu") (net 2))
 (segment (start 129.3175 96.1175) (end 154.6075 96.1175) (width 0.2) (layer "F.Cu") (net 2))
 (segment (start 182.5175 88.4) (end 164.75 88.4) (width 0.2) (layer "F.Cu") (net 10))
 (segment (start 164.75 88.4) (end 157.5325 95.6175) (width 0.2) (layer "F.Cu") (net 10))
 (segment (start 174.6425 96.6175) (end 183.005 104.98) (width 0.2) (layer "F.Cu") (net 1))
 (segment (start 157.5325 96.6175) (end 174.6425 96.6175) (width 0.2) (layer "F.Cu") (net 1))
 (segment (start 154.6075 96.6175) (end 135.7575 96.6175) (width 0.2) (layer "F.Cu") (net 9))
 (segment (start 135.7575 96.6175) (end 126.915 105.46) (width 0.2) (layer "F.Cu") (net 9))
 (segment (start 155.82 80.6925) (end 155.82 94.905) (width 0.2) (layer "F.Cu") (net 5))
 (segment (start 155.68 80.5525) (end 155.82 80.6925) (width 0.2) (layer "F.Cu") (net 5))
 (segment (start 154.6075 95.6175) (end 133.6525 95.6175) (width 0.2) (layer "F.Cu") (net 6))
 (segment (start 133.6525 95.6175) (end 126.915 88.88) (width 0.2) (layer "F.Cu") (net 6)))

